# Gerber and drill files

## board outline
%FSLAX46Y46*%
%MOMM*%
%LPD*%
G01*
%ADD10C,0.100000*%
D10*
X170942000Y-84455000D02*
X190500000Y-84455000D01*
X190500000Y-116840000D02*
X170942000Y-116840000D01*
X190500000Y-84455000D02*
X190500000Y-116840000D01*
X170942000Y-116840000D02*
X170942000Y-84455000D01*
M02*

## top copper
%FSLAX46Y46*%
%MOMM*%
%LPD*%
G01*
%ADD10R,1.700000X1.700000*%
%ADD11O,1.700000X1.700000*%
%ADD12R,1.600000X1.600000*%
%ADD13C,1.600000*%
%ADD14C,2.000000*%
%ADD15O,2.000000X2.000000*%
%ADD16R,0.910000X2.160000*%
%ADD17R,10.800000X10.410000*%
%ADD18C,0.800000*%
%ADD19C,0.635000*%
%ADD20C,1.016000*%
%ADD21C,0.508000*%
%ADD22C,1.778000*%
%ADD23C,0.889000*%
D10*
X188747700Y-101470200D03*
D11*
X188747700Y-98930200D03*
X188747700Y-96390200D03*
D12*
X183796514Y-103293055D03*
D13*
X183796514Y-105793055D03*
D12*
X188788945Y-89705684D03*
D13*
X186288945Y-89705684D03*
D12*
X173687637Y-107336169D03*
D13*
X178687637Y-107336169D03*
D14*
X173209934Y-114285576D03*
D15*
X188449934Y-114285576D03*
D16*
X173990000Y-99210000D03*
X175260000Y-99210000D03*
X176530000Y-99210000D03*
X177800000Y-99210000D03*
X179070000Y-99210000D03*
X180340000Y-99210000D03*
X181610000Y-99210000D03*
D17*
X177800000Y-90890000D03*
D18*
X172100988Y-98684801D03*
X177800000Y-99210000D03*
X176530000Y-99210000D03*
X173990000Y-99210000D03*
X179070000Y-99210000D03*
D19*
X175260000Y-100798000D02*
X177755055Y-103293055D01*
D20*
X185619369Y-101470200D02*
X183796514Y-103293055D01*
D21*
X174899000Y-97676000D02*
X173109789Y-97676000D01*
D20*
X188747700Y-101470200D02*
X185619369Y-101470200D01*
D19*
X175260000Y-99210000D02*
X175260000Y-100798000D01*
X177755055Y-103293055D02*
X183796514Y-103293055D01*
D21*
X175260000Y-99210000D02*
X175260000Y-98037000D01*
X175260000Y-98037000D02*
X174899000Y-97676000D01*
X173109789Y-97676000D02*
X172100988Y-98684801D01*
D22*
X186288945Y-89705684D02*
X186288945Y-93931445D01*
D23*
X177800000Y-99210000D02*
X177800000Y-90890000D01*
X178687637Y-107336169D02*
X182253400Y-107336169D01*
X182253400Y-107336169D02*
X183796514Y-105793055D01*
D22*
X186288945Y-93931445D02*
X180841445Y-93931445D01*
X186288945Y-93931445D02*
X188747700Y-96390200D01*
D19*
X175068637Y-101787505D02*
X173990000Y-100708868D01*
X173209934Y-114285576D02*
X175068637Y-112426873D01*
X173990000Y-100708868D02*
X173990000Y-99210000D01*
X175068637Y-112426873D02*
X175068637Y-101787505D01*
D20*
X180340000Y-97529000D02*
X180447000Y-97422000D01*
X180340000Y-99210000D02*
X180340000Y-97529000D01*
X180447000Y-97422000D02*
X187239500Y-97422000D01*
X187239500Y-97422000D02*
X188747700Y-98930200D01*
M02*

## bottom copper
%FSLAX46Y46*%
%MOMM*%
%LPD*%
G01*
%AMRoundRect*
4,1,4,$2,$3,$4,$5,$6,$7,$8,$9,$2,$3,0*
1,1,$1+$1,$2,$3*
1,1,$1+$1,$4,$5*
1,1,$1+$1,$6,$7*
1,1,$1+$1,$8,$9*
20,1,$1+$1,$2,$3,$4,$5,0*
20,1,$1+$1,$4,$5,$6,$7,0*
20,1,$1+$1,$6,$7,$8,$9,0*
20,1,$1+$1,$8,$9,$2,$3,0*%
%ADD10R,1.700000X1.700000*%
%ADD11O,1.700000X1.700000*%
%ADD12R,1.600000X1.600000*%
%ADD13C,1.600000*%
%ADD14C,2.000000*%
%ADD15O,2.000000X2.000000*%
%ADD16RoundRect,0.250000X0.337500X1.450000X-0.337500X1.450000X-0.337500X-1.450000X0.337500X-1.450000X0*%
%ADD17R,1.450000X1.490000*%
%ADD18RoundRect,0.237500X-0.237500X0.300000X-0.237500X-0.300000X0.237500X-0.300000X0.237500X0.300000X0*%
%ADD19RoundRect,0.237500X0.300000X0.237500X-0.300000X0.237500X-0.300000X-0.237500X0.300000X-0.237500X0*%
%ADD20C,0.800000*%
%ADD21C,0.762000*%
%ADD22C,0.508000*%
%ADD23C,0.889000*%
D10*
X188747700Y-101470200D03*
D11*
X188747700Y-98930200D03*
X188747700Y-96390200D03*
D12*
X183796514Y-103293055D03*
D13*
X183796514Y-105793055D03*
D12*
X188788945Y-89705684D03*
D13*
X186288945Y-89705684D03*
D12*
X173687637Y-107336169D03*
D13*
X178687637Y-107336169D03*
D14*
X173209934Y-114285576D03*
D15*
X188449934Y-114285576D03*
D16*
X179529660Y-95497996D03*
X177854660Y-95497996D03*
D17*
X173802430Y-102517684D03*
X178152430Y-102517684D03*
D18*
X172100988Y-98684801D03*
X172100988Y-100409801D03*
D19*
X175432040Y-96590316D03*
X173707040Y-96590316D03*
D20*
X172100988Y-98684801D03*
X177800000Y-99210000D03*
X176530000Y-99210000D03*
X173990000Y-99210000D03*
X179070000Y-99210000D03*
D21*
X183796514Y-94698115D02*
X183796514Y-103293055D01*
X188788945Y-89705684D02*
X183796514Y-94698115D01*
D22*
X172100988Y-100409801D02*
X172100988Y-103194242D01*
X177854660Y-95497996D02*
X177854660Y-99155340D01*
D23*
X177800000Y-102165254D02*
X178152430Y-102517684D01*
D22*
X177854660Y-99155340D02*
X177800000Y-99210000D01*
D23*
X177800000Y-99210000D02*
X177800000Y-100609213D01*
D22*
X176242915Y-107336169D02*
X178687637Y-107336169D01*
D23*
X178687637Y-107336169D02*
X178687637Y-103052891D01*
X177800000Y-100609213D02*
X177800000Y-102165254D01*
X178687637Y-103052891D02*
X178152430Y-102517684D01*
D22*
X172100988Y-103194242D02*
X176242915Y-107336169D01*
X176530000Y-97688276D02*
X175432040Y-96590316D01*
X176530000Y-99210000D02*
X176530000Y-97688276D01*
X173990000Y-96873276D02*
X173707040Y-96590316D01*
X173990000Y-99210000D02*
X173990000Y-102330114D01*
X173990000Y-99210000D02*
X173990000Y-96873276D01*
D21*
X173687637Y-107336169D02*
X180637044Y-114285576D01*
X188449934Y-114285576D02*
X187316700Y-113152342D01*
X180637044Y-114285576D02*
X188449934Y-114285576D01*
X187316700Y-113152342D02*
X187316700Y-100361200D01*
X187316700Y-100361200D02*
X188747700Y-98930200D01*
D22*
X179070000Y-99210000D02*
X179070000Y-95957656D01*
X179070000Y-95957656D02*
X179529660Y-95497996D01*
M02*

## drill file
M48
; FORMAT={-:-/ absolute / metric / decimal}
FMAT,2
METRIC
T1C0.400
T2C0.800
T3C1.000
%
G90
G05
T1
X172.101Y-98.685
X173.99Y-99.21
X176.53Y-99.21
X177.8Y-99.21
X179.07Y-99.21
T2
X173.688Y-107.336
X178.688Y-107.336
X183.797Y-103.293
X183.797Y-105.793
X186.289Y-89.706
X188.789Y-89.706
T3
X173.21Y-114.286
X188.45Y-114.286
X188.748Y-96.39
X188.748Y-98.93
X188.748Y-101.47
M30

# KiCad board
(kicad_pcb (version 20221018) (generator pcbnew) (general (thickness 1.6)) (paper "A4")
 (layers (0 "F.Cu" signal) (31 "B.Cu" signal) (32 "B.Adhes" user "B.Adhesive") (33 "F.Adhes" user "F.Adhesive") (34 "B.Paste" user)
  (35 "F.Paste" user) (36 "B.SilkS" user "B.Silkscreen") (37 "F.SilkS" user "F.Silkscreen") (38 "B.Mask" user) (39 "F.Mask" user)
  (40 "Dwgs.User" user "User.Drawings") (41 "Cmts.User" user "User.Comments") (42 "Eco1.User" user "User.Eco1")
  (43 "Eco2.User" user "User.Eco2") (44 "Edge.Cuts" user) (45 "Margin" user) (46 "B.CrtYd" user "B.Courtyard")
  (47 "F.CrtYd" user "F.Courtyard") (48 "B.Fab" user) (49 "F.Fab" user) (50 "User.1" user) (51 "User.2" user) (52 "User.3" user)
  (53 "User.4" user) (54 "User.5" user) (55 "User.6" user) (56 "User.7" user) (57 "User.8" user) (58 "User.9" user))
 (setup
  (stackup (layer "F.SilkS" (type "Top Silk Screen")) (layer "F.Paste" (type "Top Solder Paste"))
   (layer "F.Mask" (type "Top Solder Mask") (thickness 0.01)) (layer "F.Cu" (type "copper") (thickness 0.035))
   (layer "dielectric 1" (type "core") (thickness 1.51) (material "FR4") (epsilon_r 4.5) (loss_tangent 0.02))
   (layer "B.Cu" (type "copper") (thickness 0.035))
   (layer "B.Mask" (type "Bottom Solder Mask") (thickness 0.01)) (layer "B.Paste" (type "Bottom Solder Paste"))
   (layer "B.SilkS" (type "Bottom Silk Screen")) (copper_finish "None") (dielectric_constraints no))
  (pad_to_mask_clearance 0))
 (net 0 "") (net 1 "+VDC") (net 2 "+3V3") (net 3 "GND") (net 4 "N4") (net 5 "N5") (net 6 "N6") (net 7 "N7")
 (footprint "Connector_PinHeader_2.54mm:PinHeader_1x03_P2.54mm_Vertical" (layer "F.Cu") (at 188.7477 101.4702 180)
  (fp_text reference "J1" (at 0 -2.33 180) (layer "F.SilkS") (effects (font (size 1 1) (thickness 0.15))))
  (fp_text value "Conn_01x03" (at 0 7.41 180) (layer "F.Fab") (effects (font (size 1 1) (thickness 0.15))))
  (pad "1" thru_hole rect (at 0 0 180) (size 1.7 1.7) (drill 1) (layers "*.Cu" "*.Mask") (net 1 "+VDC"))
  (pad "2" thru_hole oval (at 0 2.54 180) (size 1.7 1.7) (drill 1) (layers "*.Cu" "*.Mask") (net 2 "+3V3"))
  (pad "3" thru_hole oval (at 0 5.08 180) (size 1.7 1.7) (drill 1) (layers "*.Cu" "*.Mask") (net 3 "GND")))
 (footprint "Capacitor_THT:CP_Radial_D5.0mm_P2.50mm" (layer "F.Cu") (at 183.796514 103.293055 -90)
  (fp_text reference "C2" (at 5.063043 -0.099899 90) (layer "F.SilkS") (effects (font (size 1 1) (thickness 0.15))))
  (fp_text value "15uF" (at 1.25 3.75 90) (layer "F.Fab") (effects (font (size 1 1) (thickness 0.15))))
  (pad "1" thru_hole rect (at 0 0 270) (size 1.6 1.6) (drill 0.8) (layers "*.Cu" "*.Mask") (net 1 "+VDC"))
  (pad "2" thru_hole circle (at 2.5 0 270) (size 1.6 1.6) (drill 0.8) (layers "*.Cu" "*.Mask") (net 3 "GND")))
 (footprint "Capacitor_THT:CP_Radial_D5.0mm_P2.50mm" (layer "F.Cu") (at 188.788945 89.705684 180)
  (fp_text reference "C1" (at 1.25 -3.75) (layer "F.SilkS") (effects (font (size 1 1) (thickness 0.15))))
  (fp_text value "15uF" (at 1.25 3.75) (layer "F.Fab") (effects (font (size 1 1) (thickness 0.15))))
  (pad "1" thru_hole rect (at 0 0 180) (size 1.6 1.6) (drill 0.8) (layers "*.Cu" "*.Mask") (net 1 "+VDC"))
  (pad "2" thru_hole circle (at 2.5 0 180) (size 1.6 1.6) (drill 0.8) (layers "*.Cu" "*.Mask") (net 3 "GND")))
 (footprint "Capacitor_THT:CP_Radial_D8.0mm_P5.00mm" (layer "F.Cu") (at 173.687637 107.336169)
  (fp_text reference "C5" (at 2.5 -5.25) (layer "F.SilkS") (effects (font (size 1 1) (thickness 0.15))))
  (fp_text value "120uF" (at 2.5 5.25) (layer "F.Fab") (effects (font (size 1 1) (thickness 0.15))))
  (pad "1" thru_hole rect (at 0 0) (size 1.6 1.6) (drill 0.8) (layers "*.Cu" "*.Mask") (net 2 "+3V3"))
  (pad "2" thru_hole circle (at 5 0) (size 1.6 1.6) (drill 0.8) (layers "*.Cu" "*.Mask") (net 3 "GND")))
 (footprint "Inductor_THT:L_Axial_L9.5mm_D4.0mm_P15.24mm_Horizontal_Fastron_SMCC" (layer "F.Cu") (at 173.209934 114.285576)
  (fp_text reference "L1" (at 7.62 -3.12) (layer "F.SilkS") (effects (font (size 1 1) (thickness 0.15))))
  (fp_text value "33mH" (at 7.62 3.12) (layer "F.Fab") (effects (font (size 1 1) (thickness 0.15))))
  (pad "1" thru_hole circle (at 0 0) (size 2 2) (drill 1) (layers "*.Cu" "*.Mask") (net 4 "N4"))
  (pad "2" thru_hole oval (at 15.24 0) (size 2 2) (drill 1) (layers "*.Cu" "*.Mask") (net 2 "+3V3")))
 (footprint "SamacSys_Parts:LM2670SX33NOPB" (layer "F.Cu") (at 177.8 91.44 -90)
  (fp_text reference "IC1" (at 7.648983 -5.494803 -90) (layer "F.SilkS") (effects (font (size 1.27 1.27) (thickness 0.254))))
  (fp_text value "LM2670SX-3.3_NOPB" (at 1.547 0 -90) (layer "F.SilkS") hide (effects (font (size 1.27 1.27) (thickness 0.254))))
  (pad "1" smd rect (at 7.77 3.81) (size 0.91 2.16) (layers "F.Cu" "F.Paste" "F.Mask") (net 4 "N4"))
  (pad "2" smd rect (at 7.77 2.54) (size 0.91 2.16) (layers "F.Cu" "F.Paste" "F.Mask") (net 1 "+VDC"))
  (pad "3" smd rect (at 7.77 1.27) (size 0.91 2.16) (layers "F.Cu" "F.Paste" "F.Mask") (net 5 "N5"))
  (pad "4" smd rect (at 7.77 0) (size 0.91 2.16) (layers "F.Cu" "F.Paste" "F.Mask") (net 3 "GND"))
  (pad "5" smd rect (at 7.77 -1.27) (size 0.91 2.16) (layers "F.Cu" "F.Paste" "F.Mask") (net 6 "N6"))
  (pad "6" smd rect (at 7.77 -2.54) (size 0.91 2.16) (layers "F.Cu" "F.Paste" "F.Mask") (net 2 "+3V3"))
  (pad "7" smd rect (at 7.77 -3.81) (size 0.91 2.16) (layers "F.Cu" "F.Paste" "F.Mask") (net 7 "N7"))
  (pad "8" smd rect (at -0.55 0 270) (size 10.41 10.8) (layers "F.Cu" "F.Paste" "F.Mask") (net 3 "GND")))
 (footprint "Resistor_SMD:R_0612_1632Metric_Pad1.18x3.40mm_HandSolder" (layer "B.Cu") (at 178.69216 95.497996 180)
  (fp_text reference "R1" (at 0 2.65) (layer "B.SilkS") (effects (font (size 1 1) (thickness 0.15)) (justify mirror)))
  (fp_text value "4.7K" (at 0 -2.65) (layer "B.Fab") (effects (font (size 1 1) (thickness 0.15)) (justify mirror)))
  (pad "1" smd roundrect (at -0.8375 0 180) (size 1.175 3.4) (layers "B.Cu" "B.Paste" "B.Mask") (roundrect_rratio 0.2127659574) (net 6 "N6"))
  (pad "2" smd roundrect (at 0.8375 0 180) (size 1.175 3.4) (layers "B.Cu" "B.Paste" "B.Mask") (roundrect_rratio 0.2127659574) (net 3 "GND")))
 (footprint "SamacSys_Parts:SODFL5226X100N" (layer "B.Cu") (at 175.97743 102.517684)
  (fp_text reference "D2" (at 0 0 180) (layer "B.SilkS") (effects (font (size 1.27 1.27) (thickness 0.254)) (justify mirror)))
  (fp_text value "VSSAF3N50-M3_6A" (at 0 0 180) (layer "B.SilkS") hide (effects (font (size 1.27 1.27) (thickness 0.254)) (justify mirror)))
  (pad "1" smd rect (at -2.175 0) (size 1.45 1.49) (layers "B.Cu" "B.Paste" "B.Mask") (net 4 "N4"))
  (pad "2" smd rect (at 2.175 0) (size 1.45 1.49) (layers "B.Cu" "B.Paste" "B.Mask") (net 3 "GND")))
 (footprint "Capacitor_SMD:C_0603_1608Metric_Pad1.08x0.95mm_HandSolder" (layer "B.Cu") (at 172.100988 99.547301 -90)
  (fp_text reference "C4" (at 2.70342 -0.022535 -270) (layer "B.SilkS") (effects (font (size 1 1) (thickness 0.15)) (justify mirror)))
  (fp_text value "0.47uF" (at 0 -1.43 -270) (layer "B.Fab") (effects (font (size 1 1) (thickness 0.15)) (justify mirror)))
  (pad "1" smd roundrect (at -0.8625 0 270) (size 1.075 0.95) (layers "B.Cu" "B.Paste" "B.Mask") (roundrect_rratio 0.25) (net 1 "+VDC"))
  (pad "2" smd roundrect (at 0.8625 0 270) (size 1.075 0.95) (layers "B.Cu" "B.Paste" "B.Mask") (roundrect_rratio 0.25) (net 3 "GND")))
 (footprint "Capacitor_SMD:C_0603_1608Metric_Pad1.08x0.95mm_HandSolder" (layer "B.Cu") (at 174.56954 96.590316 180)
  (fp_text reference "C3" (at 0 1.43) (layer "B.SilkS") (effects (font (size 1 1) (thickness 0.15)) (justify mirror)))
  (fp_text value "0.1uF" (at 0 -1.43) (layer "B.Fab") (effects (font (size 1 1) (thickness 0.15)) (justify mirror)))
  (pad "1" smd roundrect (at -0.8625 0 180) (size 1.075 0.95) (layers "B.Cu" "B.Paste" "B.Mask") (roundrect_rratio 0.25) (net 5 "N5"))
  (pad "2" smd roundrect (at 0.8625 0 180) (size 1.075 0.95) (layers "B.Cu" "B.Paste" "B.Mask") (roundrect_rratio 0.25) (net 4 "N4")))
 (gr_line (start 170.942 84.455) (end 190.5 84.455) (stroke (width 0.1) (type solid)) (layer "Edge.Cuts"))
 (gr_line (start 190.5 116.84) (end 170.942 116.84) (stroke (width 0.1) (type default)) (layer "Edge.Cuts"))
 (gr_line (start 190.5 84.455) (end 190.5 116.84) (stroke (width 0.1) (type default)) (layer "Edge.Cuts"))
 (gr_line (start 170.942 116.84) (end 170.942 84.455) (stroke (width 0.1) (type solid)) (layer "Edge.Cuts"))
 (segment (start 175.26 100.798) (end 177.755055 103.293055) (width 0.635) (layer "F.Cu") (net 1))
 (segment (start 185.619369 101.4702) (end 183.796514 103.293055) (width 1.016) (layer "F.Cu") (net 1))
 (segment (start 174.899 97.676) (end 173.109789 97.676) (width 0.508) (layer "F.Cu") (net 1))
 (segment (start 188.7477 101.4702) (end 185.619369 101.4702) (width 1.016) (layer "F.Cu") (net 1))
 (segment (start 175.26 99.21) (end 175.26 100.798) (width 0.635) (layer "F.Cu") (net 1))
 (segment (start 177.755055 103.293055) (end 183.796514 103.293055) (width 0.635) (layer "F.Cu") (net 1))
 (segment (start 175.26 99.21) (end 175.26 98.037) (width 0.508) (layer "F.Cu") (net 1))
 (segment (start 175.26 98.037) (end 174.899 97.676) (width 0.508) (layer "F.Cu") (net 1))
 (segment (start 173.109789 97.676) (end 172.100988 98.684801) (width 0.508) (layer "F.Cu") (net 1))
 (via (at 172.100988 98.684801) (size 0.8) (drill 0.4) (layers "F.Cu" "B.Cu") (free) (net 1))
 (segment (start 183.796514 94.698115) (end 183.796514 103.293055) (width 0.762) (layer "B.Cu") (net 1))
 (segment (start 188.788945 89.705684) (end 183.796514 94.698115) (width 0.762) (layer "B.Cu") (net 1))
 (segment (start 186.288945 89.705684) (end 186.288945 93.931445) (width 1.778) (layer "F.Cu") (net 3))
 (segment (start 177.8 99.21) (end 177.8 90.89) (width 0.889) (layer "F.Cu") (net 3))
 (segment (start 178.687637 107.336169) (end 182.2534 107.336169) (width 0.889) (layer "F.Cu") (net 3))
 (segment (start 182.2534 107.336169) (end 183.796514 105.793055) (width 0.889) (layer "F.Cu") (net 3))
 (segment (start 186.288945 93.931445) (end 180.841445 93.931445) (width 1.778) (layer "F.Cu") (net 3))
 (segment (start 186.288945 93.931445) (end 188.7477 96.3902) (width 1.778) (layer "F.Cu") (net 3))
 (via (at 177.8 99.21) (size 0.8) (drill 0.4) (layers "F.Cu" "B.Cu") (free) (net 3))
 (segment (start 172.100988 100.409801) (end 172.100988 103.194242) (width 0.508) (layer "B.Cu") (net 3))
 (segment (start 177.85466 95.497996) (end 177.85466 99.15534) (width 0.508) (layer "B.Cu") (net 3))
 (segment (start 177.8 102.165254) (end 178.15243 102.517684) (width 0.889) (layer "B.Cu") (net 3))
 (segment (start 177.85466 99.15534) (end 177.8 99.21) (width 0.508) (layer "B.Cu") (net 3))
 (segment (start 177.8 99.21) (end 177.8 100.609213) (width 0.889) (layer "B.Cu") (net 3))
 (segment (start 176.242915 107.336169) (end 178.687637 107.336169) (width 0.508) (layer "B.Cu") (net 3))
 (segment (start 178.687637 107.336169) (end 178.687637 103.052891) (width 0.889) (layer "B.Cu") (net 3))
 (segment (start 177.8 100.609213) (end 177.8 102.165254) (width 0.889) (layer "B.Cu") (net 3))
 (segment (start 178.687637 103.052891) (end 178.15243 102.517684) (width 0.889) (layer "B.Cu") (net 3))
 (segment (start 172.100988 103.194242) (end 176.242915 107.336169) (width 0.508) (layer "B.Cu") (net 3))
 (via (at 176.53 99.21) (size 0.8) (drill 0.4) (layers "F.Cu" "B.Cu") (free) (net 5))
 (segment (start 176.53 97.688276) (end 175.43204 96.590316) (width 0.508) (layer "B.Cu") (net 5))
 (segment (start 176.53 99.21) (end 176.53 97.688276) (width 0.508) (layer "B.Cu") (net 5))
 (segment (start 175.068637 101.787505) (end 173.99 100.708868) (width 0.635) (layer "F.Cu") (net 4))
 (segment (start 173.209934 114.285576) (end 175.068637 112.426873) (width 0.635) (layer "F.Cu") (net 4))
 (segment (start 173.99 100.708868) (end 173.99 99.21) (width 0.635) (layer "F.Cu") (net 4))
 (segment (start 175.068637 112.426873) (end 175.068637 101.787505) (width 0.635) (layer "F.Cu") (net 4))
 (via (at 173.99 99.21) (size 0.8) (drill 0.4) (layers "F.Cu" "B.Cu") (free) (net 4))
 (segment (start 173.99 96.873276) (end 173.70704 96.590316) (width 0.508) (layer "B.Cu") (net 4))
 (segment (start 173.99 99.21) (end 173.99 102.330114) (width 0.508) (layer "B.Cu") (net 4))
 (segment (start 173.99 99.21) (end 173.99 96.873276) (width 0.508) (layer "B.Cu") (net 4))
 (segment (start 180.34 97.529) (end 180.447 97.422) (width 1.016) (layer "F.Cu") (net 2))
 (segment (start 180.34 99.21) (end 180.34 97.529) (width 1.016) (layer "F.Cu") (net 2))
 (segment (start 180.447 97.422) (end 187.2395 97.422) (width 1.016) (layer "F.Cu") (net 2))
 (segment (start 187.2395 97.422) (end 188.7477 98.9302) (width 1.016) (layer "F.Cu") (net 2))
 (segment (start 173.687637 107.336169) (end 180.637044 114.285576) (width 0.762) (layer "B.Cu") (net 2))
 (segment (start 188.449934 114.285576) (end 187.3167 113.152342) (width 0.762) (layer "B.Cu") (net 2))
 (segment (start 180.637044 114.285576) (end 188.449934 114.285576) (width 0.762) (layer "B.Cu") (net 2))
 (segment (start 187.3167 113.152342) (end 187.3167 100.3612) (width 0.762) (layer "B.Cu") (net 2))
 (segment (start 187.3167 100.3612) (end 188.7477 98.9302) (width 0.762) (layer "B.Cu") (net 2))
 (via (at 179.07 99.21) (size 0.8) (drill 0.4) (layers "F.Cu" "B.Cu") (free) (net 6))
 (segment (start 179.07 99.21) (end 179.07 95.957656) (width 0.508) (layer "B.Cu") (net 6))
 (segment (start 179.07 95.957656) (end 179.52966 95.497996) (width 0.508) (layer "B.Cu") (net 6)))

